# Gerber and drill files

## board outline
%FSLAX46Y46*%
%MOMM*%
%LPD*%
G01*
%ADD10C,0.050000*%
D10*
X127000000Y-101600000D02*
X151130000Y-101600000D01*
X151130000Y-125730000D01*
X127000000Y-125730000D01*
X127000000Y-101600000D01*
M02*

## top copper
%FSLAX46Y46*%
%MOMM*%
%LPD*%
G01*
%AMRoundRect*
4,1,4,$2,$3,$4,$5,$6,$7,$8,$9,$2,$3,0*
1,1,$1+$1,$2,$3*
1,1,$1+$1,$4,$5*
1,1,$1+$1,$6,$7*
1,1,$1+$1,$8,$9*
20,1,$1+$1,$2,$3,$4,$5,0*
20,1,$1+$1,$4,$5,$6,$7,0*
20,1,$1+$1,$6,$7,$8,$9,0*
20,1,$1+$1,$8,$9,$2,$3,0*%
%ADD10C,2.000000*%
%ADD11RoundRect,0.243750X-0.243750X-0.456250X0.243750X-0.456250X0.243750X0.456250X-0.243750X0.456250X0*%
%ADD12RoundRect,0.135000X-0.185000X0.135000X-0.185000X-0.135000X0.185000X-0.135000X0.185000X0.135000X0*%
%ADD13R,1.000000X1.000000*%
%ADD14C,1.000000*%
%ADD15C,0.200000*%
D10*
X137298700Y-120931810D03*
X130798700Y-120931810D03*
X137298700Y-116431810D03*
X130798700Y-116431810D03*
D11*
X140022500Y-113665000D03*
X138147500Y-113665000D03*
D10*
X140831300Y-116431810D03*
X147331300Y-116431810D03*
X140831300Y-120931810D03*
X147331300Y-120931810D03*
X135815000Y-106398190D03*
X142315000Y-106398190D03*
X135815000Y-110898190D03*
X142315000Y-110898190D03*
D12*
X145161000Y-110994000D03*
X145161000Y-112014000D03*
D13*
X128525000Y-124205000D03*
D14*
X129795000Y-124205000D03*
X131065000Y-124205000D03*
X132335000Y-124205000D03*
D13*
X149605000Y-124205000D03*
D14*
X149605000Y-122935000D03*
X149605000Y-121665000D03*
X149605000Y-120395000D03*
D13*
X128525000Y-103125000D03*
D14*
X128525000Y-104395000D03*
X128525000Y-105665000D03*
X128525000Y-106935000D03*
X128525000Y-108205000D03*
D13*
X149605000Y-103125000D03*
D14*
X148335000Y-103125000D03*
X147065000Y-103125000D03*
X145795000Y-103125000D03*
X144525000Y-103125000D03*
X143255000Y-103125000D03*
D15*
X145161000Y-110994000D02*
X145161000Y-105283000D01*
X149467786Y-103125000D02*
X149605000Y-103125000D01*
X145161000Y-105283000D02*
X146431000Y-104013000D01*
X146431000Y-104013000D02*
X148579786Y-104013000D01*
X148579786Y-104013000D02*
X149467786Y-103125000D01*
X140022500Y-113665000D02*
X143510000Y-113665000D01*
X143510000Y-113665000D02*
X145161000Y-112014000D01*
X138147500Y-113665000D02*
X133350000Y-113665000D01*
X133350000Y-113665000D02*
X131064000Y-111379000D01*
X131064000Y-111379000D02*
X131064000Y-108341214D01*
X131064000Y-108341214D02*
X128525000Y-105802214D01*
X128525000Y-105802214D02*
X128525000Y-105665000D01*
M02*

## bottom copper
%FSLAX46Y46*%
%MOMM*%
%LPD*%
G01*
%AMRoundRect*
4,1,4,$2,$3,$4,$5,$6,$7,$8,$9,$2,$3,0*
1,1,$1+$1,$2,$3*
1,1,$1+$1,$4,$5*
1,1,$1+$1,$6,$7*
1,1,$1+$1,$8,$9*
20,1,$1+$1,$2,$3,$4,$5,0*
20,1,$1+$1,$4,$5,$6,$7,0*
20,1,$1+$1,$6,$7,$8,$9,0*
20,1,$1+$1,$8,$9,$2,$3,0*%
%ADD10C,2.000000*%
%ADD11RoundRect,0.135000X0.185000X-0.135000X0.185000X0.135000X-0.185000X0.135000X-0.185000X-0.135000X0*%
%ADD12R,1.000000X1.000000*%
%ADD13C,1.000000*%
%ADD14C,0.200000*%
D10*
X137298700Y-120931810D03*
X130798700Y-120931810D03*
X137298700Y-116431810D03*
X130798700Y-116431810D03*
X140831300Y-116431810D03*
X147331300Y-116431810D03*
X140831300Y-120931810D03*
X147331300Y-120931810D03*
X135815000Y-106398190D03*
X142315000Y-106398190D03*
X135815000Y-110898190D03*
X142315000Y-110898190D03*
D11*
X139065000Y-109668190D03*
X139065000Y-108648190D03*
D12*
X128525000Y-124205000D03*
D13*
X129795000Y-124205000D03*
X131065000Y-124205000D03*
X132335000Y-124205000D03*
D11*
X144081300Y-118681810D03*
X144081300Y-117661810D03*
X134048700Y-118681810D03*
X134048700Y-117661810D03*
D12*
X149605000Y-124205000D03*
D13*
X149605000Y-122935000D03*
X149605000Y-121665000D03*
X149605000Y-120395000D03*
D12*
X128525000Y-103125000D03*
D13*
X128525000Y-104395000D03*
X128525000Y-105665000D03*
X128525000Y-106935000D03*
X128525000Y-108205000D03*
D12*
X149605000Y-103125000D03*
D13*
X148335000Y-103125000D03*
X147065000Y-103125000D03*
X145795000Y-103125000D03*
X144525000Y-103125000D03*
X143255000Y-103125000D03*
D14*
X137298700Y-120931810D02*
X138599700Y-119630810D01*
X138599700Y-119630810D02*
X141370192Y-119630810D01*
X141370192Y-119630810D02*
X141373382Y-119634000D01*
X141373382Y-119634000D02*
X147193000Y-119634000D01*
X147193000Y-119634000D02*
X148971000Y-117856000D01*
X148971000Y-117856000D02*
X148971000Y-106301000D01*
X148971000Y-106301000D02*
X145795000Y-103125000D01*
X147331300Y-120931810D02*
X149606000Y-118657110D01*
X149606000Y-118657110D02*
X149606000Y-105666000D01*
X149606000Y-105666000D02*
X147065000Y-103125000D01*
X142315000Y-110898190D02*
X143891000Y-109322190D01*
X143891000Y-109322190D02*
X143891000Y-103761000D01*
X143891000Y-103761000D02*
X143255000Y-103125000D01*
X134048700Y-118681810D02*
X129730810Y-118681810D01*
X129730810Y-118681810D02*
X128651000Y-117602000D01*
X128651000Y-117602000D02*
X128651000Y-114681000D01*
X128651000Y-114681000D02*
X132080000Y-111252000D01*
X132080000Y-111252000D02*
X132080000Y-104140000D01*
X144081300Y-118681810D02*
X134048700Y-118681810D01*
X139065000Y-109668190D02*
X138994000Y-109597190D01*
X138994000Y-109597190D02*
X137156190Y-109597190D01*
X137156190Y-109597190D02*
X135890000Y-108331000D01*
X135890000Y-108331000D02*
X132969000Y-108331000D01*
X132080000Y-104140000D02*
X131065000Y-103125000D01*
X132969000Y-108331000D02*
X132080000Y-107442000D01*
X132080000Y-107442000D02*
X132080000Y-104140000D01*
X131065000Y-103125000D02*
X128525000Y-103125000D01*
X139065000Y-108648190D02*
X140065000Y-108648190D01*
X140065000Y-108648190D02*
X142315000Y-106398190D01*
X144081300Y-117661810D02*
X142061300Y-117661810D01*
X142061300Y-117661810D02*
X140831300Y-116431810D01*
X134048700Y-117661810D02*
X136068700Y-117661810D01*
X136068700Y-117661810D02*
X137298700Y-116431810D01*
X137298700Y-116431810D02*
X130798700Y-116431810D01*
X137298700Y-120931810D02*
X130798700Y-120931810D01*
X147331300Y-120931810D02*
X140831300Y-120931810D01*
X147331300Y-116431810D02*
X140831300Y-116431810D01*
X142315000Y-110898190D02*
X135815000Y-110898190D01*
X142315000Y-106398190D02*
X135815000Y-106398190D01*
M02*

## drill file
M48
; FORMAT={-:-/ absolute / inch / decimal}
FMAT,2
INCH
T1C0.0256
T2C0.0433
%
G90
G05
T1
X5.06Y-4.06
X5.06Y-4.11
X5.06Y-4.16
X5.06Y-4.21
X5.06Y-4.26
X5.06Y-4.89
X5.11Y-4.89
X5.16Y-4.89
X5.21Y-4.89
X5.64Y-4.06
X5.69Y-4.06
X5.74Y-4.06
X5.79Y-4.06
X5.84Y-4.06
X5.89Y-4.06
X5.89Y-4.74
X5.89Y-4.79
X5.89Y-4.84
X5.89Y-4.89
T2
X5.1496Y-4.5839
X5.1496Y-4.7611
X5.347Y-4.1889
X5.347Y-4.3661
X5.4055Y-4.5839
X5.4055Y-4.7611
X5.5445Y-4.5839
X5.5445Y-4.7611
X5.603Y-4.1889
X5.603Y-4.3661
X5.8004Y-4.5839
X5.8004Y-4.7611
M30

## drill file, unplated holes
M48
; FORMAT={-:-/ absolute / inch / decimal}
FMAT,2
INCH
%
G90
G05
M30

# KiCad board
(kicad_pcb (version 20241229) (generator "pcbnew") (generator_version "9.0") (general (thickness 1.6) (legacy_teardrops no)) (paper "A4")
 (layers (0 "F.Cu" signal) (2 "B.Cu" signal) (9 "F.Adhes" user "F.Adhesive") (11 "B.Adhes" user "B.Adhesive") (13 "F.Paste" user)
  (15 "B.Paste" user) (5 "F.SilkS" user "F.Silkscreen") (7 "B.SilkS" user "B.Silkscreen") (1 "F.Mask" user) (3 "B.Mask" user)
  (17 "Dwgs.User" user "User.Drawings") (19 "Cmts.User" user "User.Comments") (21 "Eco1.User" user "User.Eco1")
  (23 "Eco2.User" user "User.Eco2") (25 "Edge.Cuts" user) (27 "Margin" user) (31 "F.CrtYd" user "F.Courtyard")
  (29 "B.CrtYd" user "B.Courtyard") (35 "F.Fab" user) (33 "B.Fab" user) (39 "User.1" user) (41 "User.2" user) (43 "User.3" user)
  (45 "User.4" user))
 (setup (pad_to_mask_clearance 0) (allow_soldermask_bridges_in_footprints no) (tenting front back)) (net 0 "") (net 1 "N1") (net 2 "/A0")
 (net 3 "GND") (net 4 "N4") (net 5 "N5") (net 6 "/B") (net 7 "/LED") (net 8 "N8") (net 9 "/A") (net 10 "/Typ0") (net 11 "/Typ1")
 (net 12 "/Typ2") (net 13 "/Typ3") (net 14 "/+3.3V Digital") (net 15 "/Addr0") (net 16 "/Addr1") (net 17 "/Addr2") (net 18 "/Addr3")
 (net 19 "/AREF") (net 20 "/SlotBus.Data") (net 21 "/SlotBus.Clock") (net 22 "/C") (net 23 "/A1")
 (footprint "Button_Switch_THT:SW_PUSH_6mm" (layer "F.Cu") (at 135.815 106.39819)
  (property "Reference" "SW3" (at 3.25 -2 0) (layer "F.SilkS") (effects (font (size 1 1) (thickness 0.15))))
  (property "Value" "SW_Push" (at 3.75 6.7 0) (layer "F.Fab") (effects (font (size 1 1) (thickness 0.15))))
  (pad "1" thru_hole circle (at 0 0 90) (size 2 2) (drill 1.1) (layers "*.Cu" "*.Mask") (remove_unused_layers no) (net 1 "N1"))
  (pad "1" thru_hole circle (at 6.5 0 90) (size 2 2) (drill 1.1) (layers "*.Cu" "*.Mask") (remove_unused_layers no) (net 1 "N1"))
  (pad "2" thru_hole circle (at 0 4.5 90) (size 2 2) (drill 1.1) (layers "*.Cu" "*.Mask") (remove_unused_layers no) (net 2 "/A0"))
  (pad "2" thru_hole circle (at 6.5 4.5 90) (size 2 2) (drill 1.1) (layers "*.Cu" "*.Mask") (remove_unused_layers no) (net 2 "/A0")))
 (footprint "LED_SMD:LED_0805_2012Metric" (layer "F.Cu") (at 139.085 113.665)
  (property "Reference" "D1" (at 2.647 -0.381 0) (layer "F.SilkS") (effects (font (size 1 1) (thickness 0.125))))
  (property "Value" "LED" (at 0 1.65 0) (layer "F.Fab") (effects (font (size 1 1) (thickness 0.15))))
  (pad "1" smd roundrect (at -0.9375 0) (size 0.975 1.4) (layers "F.Cu" "F.Mask" "F.Paste") (roundrect_rratio 0.25) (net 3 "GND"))
  (pad "2" smd roundrect (at 0.9375 0) (size 0.975 1.4) (layers "F.Cu" "F.Mask" "F.Paste") (roundrect_rratio 0.25) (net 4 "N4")))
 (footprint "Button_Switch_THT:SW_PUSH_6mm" (layer "F.Cu") (at 140.8313 116.43181)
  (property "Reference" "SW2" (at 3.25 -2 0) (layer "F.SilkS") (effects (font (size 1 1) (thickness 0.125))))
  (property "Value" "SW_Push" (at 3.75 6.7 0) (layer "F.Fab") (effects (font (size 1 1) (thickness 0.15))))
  (pad "1" thru_hole circle (at 0 0 90) (size 2 2) (drill 1.1) (layers "*.Cu" "*.Mask") (remove_unused_layers no) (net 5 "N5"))
  (pad "1" thru_hole circle (at 6.5 0 90) (size 2 2) (drill 1.1) (layers "*.Cu" "*.Mask") (remove_unused_layers no) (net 5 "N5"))
  (pad "2" thru_hole circle (at 0 4.5 90) (size 2 2) (drill 1.1) (layers "*.Cu" "*.Mask") (remove_unused_layers no) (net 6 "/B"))
  (pad "2" thru_hole circle (at 6.5 4.5 90) (size 2 2) (drill 1.1) (layers "*.Cu" "*.Mask") (remove_unused_layers no) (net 6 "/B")))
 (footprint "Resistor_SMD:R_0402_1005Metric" (layer "F.Cu") (at 145.161 111.504 -90)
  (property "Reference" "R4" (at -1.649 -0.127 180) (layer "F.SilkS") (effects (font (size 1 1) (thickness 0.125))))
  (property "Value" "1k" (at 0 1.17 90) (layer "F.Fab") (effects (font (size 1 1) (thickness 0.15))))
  (pad "1" smd roundrect (at -0.51 0 270) (size 0.54 0.64) (layers "F.Cu" "F.Mask" "F.Paste") (roundrect_rratio 0.25) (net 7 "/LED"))
  (pad "2" smd roundrect (at 0.51 0 270) (size 0.54 0.64) (layers "F.Cu" "F.Mask" "F.Paste") (roundrect_rratio 0.25) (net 4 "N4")))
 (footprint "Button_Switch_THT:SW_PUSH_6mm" (layer "F.Cu") (at 130.7987 116.43181)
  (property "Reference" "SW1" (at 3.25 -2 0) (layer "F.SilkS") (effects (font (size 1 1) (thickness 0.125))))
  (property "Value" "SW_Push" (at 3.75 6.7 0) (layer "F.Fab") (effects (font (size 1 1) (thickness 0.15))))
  (pad "1" thru_hole circle (at 0 0 90) (size 2 2) (drill 1.1) (layers "*.Cu" "*.Mask") (remove_unused_layers no) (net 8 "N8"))
  (pad "1" thru_hole circle (at 6.5 0 90) (size 2 2) (drill 1.1) (layers "*.Cu" "*.Mask") (remove_unused_layers no) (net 8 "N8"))
  (pad "2" thru_hole circle (at 0 4.5 90) (size 2 2) (drill 1.1) (layers "*.Cu" "*.Mask") (remove_unused_layers no) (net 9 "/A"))
  (pad "2" thru_hole circle (at 6.5 4.5 90) (size 2 2) (drill 1.1) (layers "*.Cu" "*.Mask") (remove_unused_layers no) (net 9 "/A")))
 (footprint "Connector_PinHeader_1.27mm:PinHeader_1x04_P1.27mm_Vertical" (layer "B.Cu") (at 128.525 124.205 -90)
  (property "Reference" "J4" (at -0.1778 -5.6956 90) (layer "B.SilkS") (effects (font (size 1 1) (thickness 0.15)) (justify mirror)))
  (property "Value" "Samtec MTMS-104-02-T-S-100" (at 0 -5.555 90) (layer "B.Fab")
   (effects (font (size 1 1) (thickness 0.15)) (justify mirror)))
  (pad "1" thru_hole rect (at 0 0 270) (size 1 1) (drill 0.65) (layers "*.Cu" "*.Mask") (remove_unused_layers no) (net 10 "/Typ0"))
  (pad "2" thru_hole circle (at 0 -1.27 270) (size 1 1) (drill 0.65) (layers "*.Cu" "*.Mask") (remove_unused_layers no) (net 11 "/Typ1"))
  (pad "3" thru_hole circle (at 0 -2.54 270) (size 1 1) (drill 0.65) (layers "*.Cu" "*.Mask") (remove_unused_layers no) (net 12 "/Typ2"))
  (pad "4" thru_hole circle (at 0 -3.81 270) (size 1 1) (drill 0.65) (layers "*.Cu" "*.Mask") (remove_unused_layers no) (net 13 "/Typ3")))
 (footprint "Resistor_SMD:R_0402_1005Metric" (layer "B.Cu") (at 139.065 109.15819 90)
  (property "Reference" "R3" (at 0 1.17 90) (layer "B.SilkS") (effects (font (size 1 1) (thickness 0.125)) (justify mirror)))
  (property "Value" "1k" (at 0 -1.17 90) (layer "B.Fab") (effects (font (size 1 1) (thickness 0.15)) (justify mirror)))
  (pad "1" smd roundrect (at -0.51 0 90) (size 0.54 0.64) (layers "B.Cu" "B.Mask" "B.Paste") (roundrect_rratio 0.25)
   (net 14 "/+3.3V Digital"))
  (pad "2" smd roundrect (at 0.51 0 90) (size 0.54 0.64) (layers "B.Cu" "B.Mask" "B.Paste") (roundrect_rratio 0.25) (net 1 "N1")))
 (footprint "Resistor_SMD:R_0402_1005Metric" (layer "B.Cu") (at 144.0813 118.17181 90)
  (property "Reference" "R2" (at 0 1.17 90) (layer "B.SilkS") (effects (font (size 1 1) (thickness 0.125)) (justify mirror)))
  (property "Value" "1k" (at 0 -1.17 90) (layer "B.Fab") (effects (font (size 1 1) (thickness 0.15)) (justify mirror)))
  (pad "1" smd roundrect (at -0.51 0 90) (size 0.54 0.64) (layers "B.Cu" "B.Mask" "B.Paste") (roundrect_rratio 0.25)
   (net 14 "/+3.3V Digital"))
  (pad "2" smd roundrect (at 0.51 0 90) (size 0.54 0.64) (layers "B.Cu" "B.Mask" "B.Paste") (roundrect_rratio 0.25) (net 5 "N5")))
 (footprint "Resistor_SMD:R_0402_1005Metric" (layer "B.Cu") (at 134.0487 118.17181 90)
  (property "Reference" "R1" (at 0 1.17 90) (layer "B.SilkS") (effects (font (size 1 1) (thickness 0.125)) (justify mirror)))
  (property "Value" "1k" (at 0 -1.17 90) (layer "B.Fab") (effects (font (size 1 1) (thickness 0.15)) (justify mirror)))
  (pad "1" smd roundrect (at -0.51 0 90) (size 0.54 0.64) (layers "B.Cu" "B.Mask" "B.Paste") (roundrect_rratio 0.25)
   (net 14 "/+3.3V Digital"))
  (pad "2" smd roundrect (at 0.51 0 90) (size 0.54 0.64) (layers "B.Cu" "B.Mask" "B.Paste") (roundrect_rratio 0.25) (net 8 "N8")))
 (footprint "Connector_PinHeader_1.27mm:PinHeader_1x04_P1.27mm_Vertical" (layer "B.Cu") (at 149.605 124.205)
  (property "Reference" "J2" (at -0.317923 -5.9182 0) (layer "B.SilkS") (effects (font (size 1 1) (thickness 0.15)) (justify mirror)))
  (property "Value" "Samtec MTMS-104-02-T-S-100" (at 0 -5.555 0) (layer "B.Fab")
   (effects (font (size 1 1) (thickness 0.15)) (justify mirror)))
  (pad "1" thru_hole rect (at 0 0) (size 1 1) (drill 0.65) (layers "*.Cu" "*.Mask") (remove_unused_layers no) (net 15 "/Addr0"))
  (pad "2" thru_hole circle (at 0 -1.27) (size 1 1) (drill 0.65) (layers "*.Cu" "*.Mask") (remove_unused_layers no) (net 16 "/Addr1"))
  (pad "3" thru_hole circle (at 0 -2.54) (size 1 1) (drill 0.65) (layers "*.Cu" "*.Mask") (remove_unused_layers no) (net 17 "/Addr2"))
  (pad "4" thru_hole circle (at 0 -3.81) (size 1 1) (drill 0.65) (layers "*.Cu" "*.Mask") (remove_unused_layers no) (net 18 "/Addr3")))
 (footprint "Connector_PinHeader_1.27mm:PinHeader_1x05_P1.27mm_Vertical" (layer "B.Cu") (at 128.525 103.125 180)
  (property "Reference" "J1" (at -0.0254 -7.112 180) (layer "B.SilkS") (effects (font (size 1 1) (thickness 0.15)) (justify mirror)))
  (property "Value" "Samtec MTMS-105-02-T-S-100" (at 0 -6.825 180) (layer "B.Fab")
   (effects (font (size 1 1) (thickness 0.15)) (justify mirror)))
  (pad "1" thru_hole rect (at 0 0 180) (size 1 1) (drill 0.65) (layers "*.Cu" "*.Mask") (remove_unused_layers no) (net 14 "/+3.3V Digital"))
  (pad "2" thru_hole circle (at 0 -1.27 180) (size 1 1) (drill 0.65) (layers "*.Cu" "*.Mask") (remove_unused_layers no) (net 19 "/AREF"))
  (pad "3" thru_hole circle (at 0 -2.54 180) (size 1 1) (drill 0.65) (layers "*.Cu" "*.Mask") (remove_unused_layers no) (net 3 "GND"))
  (pad "4" thru_hole circle (at 0 -3.81 180) (size 1 1) (drill 0.65) (layers "*.Cu" "*.Mask") (remove_unused_layers no)
   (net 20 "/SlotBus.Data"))
  (pad "5" thru_hole circle (at 0 -5.08 180) (size 1 1) (drill 0.65) (layers "*.Cu" "*.Mask") (remove_unused_layers no)
   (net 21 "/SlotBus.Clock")))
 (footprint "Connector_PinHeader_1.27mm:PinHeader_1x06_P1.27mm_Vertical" (layer "B.Cu") (at 149.605 103.125 90)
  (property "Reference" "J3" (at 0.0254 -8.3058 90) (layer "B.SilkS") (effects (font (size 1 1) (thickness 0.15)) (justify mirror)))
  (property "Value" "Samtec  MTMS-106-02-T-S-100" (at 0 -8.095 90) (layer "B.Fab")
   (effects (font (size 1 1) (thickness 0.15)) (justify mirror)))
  (pad "1" thru_hole rect (at 0 0 90) (size 1 1) (drill 0.65) (layers "*.Cu" "*.Mask") (remove_unused_layers no) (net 7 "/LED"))
  (pad "2" thru_hole circle (at 0 -1.27 90) (size 1 1) (drill 0.65) (layers "*.Cu" "*.Mask") (remove_unused_layers no) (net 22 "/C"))
  (pad "3" thru_hole circle (at 0 -2.54 90) (size 1 1) (drill 0.65) (layers "*.Cu" "*.Mask") (remove_unused_layers no) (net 6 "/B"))
  (pad "4" thru_hole circle (at 0 -3.81 90) (size 1 1) (drill 0.65) (layers "*.Cu" "*.Mask") (remove_unused_layers no) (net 9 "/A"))
  (pad "5" thru_hole circle (at 0 -5.08 90) (size 1 1) (drill 0.65) (layers "*.Cu" "*.Mask") (remove_unused_layers no) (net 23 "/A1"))
  (pad "6" thru_hole circle (at 0 -6.35 90) (size 1 1) (drill 0.65) (layers "*.Cu" "*.Mask") (remove_unused_layers no) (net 2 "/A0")))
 (gr_rect (start 127 101.6) (end 151.13 125.73) (stroke (width 0.05) (type solid)) (fill no) (layer "Edge.Cuts"))
 (segment (start 131.064 108.341214) (end 128.525 105.802214) (width 0.2) (layer "F.Cu") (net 3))
 (segment (start 131.064 111.379) (end 131.064 108.341214) (width 0.2) (layer "F.Cu") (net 3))
 (segment (start 133.35 113.665) (end 131.064 111.379) (width 0.2) (layer "F.Cu") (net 3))
 (segment (start 128.525 105.802214) (end 128.525 105.665) (width 0.2) (layer "F.Cu") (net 3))
 (segment (start 138.1475 113.665) (end 133.35 113.665) (width 0.2) (layer "F.Cu") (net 3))
 (segment (start 143.51 113.665) (end 145.161 112.014) (width 0.2) (layer "F.Cu") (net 4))
 (segment (start 140.0225 113.665) (end 143.51 113.665) (width 0.2) (layer "F.Cu") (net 4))
 (segment (start 144.0813 118.68181) (end 134.0487 118.68181) (width 0.2) (layer "B.Cu") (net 14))
 (segment (start 134.0487 118.68181) (end 129.73081 118.68181) (width 0.2) (layer "B.Cu") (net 14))
 (segment (start 132.969 108.331) (end 132.08 107.442) (width 0.2) (layer "B.Cu") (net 14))
 (segment (start 137.15619 109.59719) (end 135.89 108.331) (width 0.2) (layer "B.Cu") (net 14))
 (segment (start 132.08 107.442) (end 132.08 104.14) (width 0.2) (layer "B.Cu") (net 14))
 (segment (start 129.73081 118.68181) (end 128.651 117.602) (width 0.2) (layer "B.Cu") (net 14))
 (segment (start 138.994 109.59719) (end 137.15619 109.59719) (width 0.2) (layer "B.Cu") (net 14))
 (segment (start 128.651 117.602) (end 128.651 114.681) (width 0.2) (layer "B.Cu") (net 14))
 (segment (start 139.065 109.66819) (end 138.994 109.59719) (width 0.2) (layer "B.Cu") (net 14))
 (segment (start 132.08 111.252) (end 132.08 104.14) (width 0.2) (layer "B.Cu") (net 14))
 (segment (start 132.08 104.14) (end 131.065 103.125) (width 0.2) (layer "B.Cu") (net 14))
 (segment (start 131.065 103.125) (end 128.525 103.125) (width 0.2) (layer "B.Cu") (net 14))
 (segment (start 128.651 114.681) (end 132.08 111.252) (width 0.2) (layer "B.Cu") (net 14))
 (segment (start 135.89 108.331) (end 132.969 108.331) (width 0.2) (layer "B.Cu") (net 14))
 (segment (start 147.3313 120.93181) (end 149.606 118.65711) (width 0.2) (layer "B.Cu") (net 6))
 (segment (start 147.3313 120.93181) (end 140.8313 120.93181) (width 0.2) (layer "B.Cu") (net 6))
 (segment (start 149.606 105.666) (end 147.065 103.125) (width 0.2) (layer "B.Cu") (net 6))
 (segment (start 149.606 118.65711) (end 149.606 105.666) (width 0.2) (layer "B.Cu") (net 6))
 (segment (start 146.431 104.013) (end 148.579786 104.013) (width 0.2) (layer "F.Cu") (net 7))
 (segment (start 148.579786 104.013) (end 149.467786 103.125) (width 0.2) (layer "F.Cu") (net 7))
 (segment (start 145.161 105.283) (end 146.431 104.013) (width 0.2) (layer "F.Cu") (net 7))
 (segment (start 149.467786 103.125) (end 149.605 103.125) (width 0.2) (layer "F.Cu") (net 7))
 (segment (start 145.161 110.994) (end 145.161 105.283) (width 0.2) (layer "F.Cu") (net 7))
 (segment (start 137.2987 120.93181) (end 138.5997 119.63081) (width 0.2) (layer "B.Cu") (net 9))
 (segment (start 137.2987 120.93181) (end 130.7987 120.93181) (width 0.2) (layer "B.Cu") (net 9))
 (segment (start 141.373382 119.634) (end 147.193 119.634) (width 0.2) (layer "B.Cu") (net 9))
 (segment (start 141.370192 119.63081) (end 141.373382 119.634) (width 0.2) (layer "B.Cu") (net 9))
 (segment (start 138.5997 119.63081) (end 141.370192 119.63081) (width 0.2) (layer "B.Cu") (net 9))
 (segment (start 148.971 106.301) (end 145.795 103.125) (width 0.2) (layer "B.Cu") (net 9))
 (segment (start 148.971 117.856) (end 148.971 106.301) (width 0.2) (layer "B.Cu") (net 9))
 (segment (start 147.193 119.634) (end 148.971 117.856) (width 0.2) (layer "B.Cu") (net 9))
 (segment (start 143.891 109.32219) (end 143.891 103.761) (width 0.2) (layer "B.Cu") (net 2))
 (segment (start 142.315 110.89819) (end 143.891 109.32219) (width 0.2) (layer "B.Cu") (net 2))
 (segment (start 143.891 103.761) (end 143.255 103.125) (width 0.2) (layer "B.Cu") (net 2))
 (segment (start 142.315 110.89819) (end 135.815 110.89819) (width 0.2) (layer "B.Cu") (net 2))
 (segment (start 134.0487 117.66181) (end 136.0687 117.66181) (width 0.2) (layer "B.Cu") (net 8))
 (segment (start 136.0687 117.66181) (end 137.2987 116.43181) (width 0.2) (layer "B.Cu") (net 8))
 (segment (start 137.2987 116.43181) (end 130.7987 116.43181) (width 0.2) (layer "B.Cu") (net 8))
 (segment (start 147.3313 116.43181) (end 140.8313 116.43181) (width 0.2) (layer "B.Cu") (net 5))
 (segment (start 142.0613 117.66181) (end 140.8313 116.43181) (width 0.2) (layer "B.Cu") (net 5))
 (segment (start 144.0813 117.66181) (end 142.0613 117.66181) (width 0.2) (layer "B.Cu") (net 5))
 (segment (start 140.065 108.64819) (end 142.315 106.39819) (width 0.2) (layer "B.Cu") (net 1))
 (segment (start 139.065 108.64819) (end 140.065 108.64819) (width 0.2) (layer "B.Cu") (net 1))
 (segment (start 142.315 106.39819) (end 135.815 106.39819) (width 0.2) (layer "B.Cu") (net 1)))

